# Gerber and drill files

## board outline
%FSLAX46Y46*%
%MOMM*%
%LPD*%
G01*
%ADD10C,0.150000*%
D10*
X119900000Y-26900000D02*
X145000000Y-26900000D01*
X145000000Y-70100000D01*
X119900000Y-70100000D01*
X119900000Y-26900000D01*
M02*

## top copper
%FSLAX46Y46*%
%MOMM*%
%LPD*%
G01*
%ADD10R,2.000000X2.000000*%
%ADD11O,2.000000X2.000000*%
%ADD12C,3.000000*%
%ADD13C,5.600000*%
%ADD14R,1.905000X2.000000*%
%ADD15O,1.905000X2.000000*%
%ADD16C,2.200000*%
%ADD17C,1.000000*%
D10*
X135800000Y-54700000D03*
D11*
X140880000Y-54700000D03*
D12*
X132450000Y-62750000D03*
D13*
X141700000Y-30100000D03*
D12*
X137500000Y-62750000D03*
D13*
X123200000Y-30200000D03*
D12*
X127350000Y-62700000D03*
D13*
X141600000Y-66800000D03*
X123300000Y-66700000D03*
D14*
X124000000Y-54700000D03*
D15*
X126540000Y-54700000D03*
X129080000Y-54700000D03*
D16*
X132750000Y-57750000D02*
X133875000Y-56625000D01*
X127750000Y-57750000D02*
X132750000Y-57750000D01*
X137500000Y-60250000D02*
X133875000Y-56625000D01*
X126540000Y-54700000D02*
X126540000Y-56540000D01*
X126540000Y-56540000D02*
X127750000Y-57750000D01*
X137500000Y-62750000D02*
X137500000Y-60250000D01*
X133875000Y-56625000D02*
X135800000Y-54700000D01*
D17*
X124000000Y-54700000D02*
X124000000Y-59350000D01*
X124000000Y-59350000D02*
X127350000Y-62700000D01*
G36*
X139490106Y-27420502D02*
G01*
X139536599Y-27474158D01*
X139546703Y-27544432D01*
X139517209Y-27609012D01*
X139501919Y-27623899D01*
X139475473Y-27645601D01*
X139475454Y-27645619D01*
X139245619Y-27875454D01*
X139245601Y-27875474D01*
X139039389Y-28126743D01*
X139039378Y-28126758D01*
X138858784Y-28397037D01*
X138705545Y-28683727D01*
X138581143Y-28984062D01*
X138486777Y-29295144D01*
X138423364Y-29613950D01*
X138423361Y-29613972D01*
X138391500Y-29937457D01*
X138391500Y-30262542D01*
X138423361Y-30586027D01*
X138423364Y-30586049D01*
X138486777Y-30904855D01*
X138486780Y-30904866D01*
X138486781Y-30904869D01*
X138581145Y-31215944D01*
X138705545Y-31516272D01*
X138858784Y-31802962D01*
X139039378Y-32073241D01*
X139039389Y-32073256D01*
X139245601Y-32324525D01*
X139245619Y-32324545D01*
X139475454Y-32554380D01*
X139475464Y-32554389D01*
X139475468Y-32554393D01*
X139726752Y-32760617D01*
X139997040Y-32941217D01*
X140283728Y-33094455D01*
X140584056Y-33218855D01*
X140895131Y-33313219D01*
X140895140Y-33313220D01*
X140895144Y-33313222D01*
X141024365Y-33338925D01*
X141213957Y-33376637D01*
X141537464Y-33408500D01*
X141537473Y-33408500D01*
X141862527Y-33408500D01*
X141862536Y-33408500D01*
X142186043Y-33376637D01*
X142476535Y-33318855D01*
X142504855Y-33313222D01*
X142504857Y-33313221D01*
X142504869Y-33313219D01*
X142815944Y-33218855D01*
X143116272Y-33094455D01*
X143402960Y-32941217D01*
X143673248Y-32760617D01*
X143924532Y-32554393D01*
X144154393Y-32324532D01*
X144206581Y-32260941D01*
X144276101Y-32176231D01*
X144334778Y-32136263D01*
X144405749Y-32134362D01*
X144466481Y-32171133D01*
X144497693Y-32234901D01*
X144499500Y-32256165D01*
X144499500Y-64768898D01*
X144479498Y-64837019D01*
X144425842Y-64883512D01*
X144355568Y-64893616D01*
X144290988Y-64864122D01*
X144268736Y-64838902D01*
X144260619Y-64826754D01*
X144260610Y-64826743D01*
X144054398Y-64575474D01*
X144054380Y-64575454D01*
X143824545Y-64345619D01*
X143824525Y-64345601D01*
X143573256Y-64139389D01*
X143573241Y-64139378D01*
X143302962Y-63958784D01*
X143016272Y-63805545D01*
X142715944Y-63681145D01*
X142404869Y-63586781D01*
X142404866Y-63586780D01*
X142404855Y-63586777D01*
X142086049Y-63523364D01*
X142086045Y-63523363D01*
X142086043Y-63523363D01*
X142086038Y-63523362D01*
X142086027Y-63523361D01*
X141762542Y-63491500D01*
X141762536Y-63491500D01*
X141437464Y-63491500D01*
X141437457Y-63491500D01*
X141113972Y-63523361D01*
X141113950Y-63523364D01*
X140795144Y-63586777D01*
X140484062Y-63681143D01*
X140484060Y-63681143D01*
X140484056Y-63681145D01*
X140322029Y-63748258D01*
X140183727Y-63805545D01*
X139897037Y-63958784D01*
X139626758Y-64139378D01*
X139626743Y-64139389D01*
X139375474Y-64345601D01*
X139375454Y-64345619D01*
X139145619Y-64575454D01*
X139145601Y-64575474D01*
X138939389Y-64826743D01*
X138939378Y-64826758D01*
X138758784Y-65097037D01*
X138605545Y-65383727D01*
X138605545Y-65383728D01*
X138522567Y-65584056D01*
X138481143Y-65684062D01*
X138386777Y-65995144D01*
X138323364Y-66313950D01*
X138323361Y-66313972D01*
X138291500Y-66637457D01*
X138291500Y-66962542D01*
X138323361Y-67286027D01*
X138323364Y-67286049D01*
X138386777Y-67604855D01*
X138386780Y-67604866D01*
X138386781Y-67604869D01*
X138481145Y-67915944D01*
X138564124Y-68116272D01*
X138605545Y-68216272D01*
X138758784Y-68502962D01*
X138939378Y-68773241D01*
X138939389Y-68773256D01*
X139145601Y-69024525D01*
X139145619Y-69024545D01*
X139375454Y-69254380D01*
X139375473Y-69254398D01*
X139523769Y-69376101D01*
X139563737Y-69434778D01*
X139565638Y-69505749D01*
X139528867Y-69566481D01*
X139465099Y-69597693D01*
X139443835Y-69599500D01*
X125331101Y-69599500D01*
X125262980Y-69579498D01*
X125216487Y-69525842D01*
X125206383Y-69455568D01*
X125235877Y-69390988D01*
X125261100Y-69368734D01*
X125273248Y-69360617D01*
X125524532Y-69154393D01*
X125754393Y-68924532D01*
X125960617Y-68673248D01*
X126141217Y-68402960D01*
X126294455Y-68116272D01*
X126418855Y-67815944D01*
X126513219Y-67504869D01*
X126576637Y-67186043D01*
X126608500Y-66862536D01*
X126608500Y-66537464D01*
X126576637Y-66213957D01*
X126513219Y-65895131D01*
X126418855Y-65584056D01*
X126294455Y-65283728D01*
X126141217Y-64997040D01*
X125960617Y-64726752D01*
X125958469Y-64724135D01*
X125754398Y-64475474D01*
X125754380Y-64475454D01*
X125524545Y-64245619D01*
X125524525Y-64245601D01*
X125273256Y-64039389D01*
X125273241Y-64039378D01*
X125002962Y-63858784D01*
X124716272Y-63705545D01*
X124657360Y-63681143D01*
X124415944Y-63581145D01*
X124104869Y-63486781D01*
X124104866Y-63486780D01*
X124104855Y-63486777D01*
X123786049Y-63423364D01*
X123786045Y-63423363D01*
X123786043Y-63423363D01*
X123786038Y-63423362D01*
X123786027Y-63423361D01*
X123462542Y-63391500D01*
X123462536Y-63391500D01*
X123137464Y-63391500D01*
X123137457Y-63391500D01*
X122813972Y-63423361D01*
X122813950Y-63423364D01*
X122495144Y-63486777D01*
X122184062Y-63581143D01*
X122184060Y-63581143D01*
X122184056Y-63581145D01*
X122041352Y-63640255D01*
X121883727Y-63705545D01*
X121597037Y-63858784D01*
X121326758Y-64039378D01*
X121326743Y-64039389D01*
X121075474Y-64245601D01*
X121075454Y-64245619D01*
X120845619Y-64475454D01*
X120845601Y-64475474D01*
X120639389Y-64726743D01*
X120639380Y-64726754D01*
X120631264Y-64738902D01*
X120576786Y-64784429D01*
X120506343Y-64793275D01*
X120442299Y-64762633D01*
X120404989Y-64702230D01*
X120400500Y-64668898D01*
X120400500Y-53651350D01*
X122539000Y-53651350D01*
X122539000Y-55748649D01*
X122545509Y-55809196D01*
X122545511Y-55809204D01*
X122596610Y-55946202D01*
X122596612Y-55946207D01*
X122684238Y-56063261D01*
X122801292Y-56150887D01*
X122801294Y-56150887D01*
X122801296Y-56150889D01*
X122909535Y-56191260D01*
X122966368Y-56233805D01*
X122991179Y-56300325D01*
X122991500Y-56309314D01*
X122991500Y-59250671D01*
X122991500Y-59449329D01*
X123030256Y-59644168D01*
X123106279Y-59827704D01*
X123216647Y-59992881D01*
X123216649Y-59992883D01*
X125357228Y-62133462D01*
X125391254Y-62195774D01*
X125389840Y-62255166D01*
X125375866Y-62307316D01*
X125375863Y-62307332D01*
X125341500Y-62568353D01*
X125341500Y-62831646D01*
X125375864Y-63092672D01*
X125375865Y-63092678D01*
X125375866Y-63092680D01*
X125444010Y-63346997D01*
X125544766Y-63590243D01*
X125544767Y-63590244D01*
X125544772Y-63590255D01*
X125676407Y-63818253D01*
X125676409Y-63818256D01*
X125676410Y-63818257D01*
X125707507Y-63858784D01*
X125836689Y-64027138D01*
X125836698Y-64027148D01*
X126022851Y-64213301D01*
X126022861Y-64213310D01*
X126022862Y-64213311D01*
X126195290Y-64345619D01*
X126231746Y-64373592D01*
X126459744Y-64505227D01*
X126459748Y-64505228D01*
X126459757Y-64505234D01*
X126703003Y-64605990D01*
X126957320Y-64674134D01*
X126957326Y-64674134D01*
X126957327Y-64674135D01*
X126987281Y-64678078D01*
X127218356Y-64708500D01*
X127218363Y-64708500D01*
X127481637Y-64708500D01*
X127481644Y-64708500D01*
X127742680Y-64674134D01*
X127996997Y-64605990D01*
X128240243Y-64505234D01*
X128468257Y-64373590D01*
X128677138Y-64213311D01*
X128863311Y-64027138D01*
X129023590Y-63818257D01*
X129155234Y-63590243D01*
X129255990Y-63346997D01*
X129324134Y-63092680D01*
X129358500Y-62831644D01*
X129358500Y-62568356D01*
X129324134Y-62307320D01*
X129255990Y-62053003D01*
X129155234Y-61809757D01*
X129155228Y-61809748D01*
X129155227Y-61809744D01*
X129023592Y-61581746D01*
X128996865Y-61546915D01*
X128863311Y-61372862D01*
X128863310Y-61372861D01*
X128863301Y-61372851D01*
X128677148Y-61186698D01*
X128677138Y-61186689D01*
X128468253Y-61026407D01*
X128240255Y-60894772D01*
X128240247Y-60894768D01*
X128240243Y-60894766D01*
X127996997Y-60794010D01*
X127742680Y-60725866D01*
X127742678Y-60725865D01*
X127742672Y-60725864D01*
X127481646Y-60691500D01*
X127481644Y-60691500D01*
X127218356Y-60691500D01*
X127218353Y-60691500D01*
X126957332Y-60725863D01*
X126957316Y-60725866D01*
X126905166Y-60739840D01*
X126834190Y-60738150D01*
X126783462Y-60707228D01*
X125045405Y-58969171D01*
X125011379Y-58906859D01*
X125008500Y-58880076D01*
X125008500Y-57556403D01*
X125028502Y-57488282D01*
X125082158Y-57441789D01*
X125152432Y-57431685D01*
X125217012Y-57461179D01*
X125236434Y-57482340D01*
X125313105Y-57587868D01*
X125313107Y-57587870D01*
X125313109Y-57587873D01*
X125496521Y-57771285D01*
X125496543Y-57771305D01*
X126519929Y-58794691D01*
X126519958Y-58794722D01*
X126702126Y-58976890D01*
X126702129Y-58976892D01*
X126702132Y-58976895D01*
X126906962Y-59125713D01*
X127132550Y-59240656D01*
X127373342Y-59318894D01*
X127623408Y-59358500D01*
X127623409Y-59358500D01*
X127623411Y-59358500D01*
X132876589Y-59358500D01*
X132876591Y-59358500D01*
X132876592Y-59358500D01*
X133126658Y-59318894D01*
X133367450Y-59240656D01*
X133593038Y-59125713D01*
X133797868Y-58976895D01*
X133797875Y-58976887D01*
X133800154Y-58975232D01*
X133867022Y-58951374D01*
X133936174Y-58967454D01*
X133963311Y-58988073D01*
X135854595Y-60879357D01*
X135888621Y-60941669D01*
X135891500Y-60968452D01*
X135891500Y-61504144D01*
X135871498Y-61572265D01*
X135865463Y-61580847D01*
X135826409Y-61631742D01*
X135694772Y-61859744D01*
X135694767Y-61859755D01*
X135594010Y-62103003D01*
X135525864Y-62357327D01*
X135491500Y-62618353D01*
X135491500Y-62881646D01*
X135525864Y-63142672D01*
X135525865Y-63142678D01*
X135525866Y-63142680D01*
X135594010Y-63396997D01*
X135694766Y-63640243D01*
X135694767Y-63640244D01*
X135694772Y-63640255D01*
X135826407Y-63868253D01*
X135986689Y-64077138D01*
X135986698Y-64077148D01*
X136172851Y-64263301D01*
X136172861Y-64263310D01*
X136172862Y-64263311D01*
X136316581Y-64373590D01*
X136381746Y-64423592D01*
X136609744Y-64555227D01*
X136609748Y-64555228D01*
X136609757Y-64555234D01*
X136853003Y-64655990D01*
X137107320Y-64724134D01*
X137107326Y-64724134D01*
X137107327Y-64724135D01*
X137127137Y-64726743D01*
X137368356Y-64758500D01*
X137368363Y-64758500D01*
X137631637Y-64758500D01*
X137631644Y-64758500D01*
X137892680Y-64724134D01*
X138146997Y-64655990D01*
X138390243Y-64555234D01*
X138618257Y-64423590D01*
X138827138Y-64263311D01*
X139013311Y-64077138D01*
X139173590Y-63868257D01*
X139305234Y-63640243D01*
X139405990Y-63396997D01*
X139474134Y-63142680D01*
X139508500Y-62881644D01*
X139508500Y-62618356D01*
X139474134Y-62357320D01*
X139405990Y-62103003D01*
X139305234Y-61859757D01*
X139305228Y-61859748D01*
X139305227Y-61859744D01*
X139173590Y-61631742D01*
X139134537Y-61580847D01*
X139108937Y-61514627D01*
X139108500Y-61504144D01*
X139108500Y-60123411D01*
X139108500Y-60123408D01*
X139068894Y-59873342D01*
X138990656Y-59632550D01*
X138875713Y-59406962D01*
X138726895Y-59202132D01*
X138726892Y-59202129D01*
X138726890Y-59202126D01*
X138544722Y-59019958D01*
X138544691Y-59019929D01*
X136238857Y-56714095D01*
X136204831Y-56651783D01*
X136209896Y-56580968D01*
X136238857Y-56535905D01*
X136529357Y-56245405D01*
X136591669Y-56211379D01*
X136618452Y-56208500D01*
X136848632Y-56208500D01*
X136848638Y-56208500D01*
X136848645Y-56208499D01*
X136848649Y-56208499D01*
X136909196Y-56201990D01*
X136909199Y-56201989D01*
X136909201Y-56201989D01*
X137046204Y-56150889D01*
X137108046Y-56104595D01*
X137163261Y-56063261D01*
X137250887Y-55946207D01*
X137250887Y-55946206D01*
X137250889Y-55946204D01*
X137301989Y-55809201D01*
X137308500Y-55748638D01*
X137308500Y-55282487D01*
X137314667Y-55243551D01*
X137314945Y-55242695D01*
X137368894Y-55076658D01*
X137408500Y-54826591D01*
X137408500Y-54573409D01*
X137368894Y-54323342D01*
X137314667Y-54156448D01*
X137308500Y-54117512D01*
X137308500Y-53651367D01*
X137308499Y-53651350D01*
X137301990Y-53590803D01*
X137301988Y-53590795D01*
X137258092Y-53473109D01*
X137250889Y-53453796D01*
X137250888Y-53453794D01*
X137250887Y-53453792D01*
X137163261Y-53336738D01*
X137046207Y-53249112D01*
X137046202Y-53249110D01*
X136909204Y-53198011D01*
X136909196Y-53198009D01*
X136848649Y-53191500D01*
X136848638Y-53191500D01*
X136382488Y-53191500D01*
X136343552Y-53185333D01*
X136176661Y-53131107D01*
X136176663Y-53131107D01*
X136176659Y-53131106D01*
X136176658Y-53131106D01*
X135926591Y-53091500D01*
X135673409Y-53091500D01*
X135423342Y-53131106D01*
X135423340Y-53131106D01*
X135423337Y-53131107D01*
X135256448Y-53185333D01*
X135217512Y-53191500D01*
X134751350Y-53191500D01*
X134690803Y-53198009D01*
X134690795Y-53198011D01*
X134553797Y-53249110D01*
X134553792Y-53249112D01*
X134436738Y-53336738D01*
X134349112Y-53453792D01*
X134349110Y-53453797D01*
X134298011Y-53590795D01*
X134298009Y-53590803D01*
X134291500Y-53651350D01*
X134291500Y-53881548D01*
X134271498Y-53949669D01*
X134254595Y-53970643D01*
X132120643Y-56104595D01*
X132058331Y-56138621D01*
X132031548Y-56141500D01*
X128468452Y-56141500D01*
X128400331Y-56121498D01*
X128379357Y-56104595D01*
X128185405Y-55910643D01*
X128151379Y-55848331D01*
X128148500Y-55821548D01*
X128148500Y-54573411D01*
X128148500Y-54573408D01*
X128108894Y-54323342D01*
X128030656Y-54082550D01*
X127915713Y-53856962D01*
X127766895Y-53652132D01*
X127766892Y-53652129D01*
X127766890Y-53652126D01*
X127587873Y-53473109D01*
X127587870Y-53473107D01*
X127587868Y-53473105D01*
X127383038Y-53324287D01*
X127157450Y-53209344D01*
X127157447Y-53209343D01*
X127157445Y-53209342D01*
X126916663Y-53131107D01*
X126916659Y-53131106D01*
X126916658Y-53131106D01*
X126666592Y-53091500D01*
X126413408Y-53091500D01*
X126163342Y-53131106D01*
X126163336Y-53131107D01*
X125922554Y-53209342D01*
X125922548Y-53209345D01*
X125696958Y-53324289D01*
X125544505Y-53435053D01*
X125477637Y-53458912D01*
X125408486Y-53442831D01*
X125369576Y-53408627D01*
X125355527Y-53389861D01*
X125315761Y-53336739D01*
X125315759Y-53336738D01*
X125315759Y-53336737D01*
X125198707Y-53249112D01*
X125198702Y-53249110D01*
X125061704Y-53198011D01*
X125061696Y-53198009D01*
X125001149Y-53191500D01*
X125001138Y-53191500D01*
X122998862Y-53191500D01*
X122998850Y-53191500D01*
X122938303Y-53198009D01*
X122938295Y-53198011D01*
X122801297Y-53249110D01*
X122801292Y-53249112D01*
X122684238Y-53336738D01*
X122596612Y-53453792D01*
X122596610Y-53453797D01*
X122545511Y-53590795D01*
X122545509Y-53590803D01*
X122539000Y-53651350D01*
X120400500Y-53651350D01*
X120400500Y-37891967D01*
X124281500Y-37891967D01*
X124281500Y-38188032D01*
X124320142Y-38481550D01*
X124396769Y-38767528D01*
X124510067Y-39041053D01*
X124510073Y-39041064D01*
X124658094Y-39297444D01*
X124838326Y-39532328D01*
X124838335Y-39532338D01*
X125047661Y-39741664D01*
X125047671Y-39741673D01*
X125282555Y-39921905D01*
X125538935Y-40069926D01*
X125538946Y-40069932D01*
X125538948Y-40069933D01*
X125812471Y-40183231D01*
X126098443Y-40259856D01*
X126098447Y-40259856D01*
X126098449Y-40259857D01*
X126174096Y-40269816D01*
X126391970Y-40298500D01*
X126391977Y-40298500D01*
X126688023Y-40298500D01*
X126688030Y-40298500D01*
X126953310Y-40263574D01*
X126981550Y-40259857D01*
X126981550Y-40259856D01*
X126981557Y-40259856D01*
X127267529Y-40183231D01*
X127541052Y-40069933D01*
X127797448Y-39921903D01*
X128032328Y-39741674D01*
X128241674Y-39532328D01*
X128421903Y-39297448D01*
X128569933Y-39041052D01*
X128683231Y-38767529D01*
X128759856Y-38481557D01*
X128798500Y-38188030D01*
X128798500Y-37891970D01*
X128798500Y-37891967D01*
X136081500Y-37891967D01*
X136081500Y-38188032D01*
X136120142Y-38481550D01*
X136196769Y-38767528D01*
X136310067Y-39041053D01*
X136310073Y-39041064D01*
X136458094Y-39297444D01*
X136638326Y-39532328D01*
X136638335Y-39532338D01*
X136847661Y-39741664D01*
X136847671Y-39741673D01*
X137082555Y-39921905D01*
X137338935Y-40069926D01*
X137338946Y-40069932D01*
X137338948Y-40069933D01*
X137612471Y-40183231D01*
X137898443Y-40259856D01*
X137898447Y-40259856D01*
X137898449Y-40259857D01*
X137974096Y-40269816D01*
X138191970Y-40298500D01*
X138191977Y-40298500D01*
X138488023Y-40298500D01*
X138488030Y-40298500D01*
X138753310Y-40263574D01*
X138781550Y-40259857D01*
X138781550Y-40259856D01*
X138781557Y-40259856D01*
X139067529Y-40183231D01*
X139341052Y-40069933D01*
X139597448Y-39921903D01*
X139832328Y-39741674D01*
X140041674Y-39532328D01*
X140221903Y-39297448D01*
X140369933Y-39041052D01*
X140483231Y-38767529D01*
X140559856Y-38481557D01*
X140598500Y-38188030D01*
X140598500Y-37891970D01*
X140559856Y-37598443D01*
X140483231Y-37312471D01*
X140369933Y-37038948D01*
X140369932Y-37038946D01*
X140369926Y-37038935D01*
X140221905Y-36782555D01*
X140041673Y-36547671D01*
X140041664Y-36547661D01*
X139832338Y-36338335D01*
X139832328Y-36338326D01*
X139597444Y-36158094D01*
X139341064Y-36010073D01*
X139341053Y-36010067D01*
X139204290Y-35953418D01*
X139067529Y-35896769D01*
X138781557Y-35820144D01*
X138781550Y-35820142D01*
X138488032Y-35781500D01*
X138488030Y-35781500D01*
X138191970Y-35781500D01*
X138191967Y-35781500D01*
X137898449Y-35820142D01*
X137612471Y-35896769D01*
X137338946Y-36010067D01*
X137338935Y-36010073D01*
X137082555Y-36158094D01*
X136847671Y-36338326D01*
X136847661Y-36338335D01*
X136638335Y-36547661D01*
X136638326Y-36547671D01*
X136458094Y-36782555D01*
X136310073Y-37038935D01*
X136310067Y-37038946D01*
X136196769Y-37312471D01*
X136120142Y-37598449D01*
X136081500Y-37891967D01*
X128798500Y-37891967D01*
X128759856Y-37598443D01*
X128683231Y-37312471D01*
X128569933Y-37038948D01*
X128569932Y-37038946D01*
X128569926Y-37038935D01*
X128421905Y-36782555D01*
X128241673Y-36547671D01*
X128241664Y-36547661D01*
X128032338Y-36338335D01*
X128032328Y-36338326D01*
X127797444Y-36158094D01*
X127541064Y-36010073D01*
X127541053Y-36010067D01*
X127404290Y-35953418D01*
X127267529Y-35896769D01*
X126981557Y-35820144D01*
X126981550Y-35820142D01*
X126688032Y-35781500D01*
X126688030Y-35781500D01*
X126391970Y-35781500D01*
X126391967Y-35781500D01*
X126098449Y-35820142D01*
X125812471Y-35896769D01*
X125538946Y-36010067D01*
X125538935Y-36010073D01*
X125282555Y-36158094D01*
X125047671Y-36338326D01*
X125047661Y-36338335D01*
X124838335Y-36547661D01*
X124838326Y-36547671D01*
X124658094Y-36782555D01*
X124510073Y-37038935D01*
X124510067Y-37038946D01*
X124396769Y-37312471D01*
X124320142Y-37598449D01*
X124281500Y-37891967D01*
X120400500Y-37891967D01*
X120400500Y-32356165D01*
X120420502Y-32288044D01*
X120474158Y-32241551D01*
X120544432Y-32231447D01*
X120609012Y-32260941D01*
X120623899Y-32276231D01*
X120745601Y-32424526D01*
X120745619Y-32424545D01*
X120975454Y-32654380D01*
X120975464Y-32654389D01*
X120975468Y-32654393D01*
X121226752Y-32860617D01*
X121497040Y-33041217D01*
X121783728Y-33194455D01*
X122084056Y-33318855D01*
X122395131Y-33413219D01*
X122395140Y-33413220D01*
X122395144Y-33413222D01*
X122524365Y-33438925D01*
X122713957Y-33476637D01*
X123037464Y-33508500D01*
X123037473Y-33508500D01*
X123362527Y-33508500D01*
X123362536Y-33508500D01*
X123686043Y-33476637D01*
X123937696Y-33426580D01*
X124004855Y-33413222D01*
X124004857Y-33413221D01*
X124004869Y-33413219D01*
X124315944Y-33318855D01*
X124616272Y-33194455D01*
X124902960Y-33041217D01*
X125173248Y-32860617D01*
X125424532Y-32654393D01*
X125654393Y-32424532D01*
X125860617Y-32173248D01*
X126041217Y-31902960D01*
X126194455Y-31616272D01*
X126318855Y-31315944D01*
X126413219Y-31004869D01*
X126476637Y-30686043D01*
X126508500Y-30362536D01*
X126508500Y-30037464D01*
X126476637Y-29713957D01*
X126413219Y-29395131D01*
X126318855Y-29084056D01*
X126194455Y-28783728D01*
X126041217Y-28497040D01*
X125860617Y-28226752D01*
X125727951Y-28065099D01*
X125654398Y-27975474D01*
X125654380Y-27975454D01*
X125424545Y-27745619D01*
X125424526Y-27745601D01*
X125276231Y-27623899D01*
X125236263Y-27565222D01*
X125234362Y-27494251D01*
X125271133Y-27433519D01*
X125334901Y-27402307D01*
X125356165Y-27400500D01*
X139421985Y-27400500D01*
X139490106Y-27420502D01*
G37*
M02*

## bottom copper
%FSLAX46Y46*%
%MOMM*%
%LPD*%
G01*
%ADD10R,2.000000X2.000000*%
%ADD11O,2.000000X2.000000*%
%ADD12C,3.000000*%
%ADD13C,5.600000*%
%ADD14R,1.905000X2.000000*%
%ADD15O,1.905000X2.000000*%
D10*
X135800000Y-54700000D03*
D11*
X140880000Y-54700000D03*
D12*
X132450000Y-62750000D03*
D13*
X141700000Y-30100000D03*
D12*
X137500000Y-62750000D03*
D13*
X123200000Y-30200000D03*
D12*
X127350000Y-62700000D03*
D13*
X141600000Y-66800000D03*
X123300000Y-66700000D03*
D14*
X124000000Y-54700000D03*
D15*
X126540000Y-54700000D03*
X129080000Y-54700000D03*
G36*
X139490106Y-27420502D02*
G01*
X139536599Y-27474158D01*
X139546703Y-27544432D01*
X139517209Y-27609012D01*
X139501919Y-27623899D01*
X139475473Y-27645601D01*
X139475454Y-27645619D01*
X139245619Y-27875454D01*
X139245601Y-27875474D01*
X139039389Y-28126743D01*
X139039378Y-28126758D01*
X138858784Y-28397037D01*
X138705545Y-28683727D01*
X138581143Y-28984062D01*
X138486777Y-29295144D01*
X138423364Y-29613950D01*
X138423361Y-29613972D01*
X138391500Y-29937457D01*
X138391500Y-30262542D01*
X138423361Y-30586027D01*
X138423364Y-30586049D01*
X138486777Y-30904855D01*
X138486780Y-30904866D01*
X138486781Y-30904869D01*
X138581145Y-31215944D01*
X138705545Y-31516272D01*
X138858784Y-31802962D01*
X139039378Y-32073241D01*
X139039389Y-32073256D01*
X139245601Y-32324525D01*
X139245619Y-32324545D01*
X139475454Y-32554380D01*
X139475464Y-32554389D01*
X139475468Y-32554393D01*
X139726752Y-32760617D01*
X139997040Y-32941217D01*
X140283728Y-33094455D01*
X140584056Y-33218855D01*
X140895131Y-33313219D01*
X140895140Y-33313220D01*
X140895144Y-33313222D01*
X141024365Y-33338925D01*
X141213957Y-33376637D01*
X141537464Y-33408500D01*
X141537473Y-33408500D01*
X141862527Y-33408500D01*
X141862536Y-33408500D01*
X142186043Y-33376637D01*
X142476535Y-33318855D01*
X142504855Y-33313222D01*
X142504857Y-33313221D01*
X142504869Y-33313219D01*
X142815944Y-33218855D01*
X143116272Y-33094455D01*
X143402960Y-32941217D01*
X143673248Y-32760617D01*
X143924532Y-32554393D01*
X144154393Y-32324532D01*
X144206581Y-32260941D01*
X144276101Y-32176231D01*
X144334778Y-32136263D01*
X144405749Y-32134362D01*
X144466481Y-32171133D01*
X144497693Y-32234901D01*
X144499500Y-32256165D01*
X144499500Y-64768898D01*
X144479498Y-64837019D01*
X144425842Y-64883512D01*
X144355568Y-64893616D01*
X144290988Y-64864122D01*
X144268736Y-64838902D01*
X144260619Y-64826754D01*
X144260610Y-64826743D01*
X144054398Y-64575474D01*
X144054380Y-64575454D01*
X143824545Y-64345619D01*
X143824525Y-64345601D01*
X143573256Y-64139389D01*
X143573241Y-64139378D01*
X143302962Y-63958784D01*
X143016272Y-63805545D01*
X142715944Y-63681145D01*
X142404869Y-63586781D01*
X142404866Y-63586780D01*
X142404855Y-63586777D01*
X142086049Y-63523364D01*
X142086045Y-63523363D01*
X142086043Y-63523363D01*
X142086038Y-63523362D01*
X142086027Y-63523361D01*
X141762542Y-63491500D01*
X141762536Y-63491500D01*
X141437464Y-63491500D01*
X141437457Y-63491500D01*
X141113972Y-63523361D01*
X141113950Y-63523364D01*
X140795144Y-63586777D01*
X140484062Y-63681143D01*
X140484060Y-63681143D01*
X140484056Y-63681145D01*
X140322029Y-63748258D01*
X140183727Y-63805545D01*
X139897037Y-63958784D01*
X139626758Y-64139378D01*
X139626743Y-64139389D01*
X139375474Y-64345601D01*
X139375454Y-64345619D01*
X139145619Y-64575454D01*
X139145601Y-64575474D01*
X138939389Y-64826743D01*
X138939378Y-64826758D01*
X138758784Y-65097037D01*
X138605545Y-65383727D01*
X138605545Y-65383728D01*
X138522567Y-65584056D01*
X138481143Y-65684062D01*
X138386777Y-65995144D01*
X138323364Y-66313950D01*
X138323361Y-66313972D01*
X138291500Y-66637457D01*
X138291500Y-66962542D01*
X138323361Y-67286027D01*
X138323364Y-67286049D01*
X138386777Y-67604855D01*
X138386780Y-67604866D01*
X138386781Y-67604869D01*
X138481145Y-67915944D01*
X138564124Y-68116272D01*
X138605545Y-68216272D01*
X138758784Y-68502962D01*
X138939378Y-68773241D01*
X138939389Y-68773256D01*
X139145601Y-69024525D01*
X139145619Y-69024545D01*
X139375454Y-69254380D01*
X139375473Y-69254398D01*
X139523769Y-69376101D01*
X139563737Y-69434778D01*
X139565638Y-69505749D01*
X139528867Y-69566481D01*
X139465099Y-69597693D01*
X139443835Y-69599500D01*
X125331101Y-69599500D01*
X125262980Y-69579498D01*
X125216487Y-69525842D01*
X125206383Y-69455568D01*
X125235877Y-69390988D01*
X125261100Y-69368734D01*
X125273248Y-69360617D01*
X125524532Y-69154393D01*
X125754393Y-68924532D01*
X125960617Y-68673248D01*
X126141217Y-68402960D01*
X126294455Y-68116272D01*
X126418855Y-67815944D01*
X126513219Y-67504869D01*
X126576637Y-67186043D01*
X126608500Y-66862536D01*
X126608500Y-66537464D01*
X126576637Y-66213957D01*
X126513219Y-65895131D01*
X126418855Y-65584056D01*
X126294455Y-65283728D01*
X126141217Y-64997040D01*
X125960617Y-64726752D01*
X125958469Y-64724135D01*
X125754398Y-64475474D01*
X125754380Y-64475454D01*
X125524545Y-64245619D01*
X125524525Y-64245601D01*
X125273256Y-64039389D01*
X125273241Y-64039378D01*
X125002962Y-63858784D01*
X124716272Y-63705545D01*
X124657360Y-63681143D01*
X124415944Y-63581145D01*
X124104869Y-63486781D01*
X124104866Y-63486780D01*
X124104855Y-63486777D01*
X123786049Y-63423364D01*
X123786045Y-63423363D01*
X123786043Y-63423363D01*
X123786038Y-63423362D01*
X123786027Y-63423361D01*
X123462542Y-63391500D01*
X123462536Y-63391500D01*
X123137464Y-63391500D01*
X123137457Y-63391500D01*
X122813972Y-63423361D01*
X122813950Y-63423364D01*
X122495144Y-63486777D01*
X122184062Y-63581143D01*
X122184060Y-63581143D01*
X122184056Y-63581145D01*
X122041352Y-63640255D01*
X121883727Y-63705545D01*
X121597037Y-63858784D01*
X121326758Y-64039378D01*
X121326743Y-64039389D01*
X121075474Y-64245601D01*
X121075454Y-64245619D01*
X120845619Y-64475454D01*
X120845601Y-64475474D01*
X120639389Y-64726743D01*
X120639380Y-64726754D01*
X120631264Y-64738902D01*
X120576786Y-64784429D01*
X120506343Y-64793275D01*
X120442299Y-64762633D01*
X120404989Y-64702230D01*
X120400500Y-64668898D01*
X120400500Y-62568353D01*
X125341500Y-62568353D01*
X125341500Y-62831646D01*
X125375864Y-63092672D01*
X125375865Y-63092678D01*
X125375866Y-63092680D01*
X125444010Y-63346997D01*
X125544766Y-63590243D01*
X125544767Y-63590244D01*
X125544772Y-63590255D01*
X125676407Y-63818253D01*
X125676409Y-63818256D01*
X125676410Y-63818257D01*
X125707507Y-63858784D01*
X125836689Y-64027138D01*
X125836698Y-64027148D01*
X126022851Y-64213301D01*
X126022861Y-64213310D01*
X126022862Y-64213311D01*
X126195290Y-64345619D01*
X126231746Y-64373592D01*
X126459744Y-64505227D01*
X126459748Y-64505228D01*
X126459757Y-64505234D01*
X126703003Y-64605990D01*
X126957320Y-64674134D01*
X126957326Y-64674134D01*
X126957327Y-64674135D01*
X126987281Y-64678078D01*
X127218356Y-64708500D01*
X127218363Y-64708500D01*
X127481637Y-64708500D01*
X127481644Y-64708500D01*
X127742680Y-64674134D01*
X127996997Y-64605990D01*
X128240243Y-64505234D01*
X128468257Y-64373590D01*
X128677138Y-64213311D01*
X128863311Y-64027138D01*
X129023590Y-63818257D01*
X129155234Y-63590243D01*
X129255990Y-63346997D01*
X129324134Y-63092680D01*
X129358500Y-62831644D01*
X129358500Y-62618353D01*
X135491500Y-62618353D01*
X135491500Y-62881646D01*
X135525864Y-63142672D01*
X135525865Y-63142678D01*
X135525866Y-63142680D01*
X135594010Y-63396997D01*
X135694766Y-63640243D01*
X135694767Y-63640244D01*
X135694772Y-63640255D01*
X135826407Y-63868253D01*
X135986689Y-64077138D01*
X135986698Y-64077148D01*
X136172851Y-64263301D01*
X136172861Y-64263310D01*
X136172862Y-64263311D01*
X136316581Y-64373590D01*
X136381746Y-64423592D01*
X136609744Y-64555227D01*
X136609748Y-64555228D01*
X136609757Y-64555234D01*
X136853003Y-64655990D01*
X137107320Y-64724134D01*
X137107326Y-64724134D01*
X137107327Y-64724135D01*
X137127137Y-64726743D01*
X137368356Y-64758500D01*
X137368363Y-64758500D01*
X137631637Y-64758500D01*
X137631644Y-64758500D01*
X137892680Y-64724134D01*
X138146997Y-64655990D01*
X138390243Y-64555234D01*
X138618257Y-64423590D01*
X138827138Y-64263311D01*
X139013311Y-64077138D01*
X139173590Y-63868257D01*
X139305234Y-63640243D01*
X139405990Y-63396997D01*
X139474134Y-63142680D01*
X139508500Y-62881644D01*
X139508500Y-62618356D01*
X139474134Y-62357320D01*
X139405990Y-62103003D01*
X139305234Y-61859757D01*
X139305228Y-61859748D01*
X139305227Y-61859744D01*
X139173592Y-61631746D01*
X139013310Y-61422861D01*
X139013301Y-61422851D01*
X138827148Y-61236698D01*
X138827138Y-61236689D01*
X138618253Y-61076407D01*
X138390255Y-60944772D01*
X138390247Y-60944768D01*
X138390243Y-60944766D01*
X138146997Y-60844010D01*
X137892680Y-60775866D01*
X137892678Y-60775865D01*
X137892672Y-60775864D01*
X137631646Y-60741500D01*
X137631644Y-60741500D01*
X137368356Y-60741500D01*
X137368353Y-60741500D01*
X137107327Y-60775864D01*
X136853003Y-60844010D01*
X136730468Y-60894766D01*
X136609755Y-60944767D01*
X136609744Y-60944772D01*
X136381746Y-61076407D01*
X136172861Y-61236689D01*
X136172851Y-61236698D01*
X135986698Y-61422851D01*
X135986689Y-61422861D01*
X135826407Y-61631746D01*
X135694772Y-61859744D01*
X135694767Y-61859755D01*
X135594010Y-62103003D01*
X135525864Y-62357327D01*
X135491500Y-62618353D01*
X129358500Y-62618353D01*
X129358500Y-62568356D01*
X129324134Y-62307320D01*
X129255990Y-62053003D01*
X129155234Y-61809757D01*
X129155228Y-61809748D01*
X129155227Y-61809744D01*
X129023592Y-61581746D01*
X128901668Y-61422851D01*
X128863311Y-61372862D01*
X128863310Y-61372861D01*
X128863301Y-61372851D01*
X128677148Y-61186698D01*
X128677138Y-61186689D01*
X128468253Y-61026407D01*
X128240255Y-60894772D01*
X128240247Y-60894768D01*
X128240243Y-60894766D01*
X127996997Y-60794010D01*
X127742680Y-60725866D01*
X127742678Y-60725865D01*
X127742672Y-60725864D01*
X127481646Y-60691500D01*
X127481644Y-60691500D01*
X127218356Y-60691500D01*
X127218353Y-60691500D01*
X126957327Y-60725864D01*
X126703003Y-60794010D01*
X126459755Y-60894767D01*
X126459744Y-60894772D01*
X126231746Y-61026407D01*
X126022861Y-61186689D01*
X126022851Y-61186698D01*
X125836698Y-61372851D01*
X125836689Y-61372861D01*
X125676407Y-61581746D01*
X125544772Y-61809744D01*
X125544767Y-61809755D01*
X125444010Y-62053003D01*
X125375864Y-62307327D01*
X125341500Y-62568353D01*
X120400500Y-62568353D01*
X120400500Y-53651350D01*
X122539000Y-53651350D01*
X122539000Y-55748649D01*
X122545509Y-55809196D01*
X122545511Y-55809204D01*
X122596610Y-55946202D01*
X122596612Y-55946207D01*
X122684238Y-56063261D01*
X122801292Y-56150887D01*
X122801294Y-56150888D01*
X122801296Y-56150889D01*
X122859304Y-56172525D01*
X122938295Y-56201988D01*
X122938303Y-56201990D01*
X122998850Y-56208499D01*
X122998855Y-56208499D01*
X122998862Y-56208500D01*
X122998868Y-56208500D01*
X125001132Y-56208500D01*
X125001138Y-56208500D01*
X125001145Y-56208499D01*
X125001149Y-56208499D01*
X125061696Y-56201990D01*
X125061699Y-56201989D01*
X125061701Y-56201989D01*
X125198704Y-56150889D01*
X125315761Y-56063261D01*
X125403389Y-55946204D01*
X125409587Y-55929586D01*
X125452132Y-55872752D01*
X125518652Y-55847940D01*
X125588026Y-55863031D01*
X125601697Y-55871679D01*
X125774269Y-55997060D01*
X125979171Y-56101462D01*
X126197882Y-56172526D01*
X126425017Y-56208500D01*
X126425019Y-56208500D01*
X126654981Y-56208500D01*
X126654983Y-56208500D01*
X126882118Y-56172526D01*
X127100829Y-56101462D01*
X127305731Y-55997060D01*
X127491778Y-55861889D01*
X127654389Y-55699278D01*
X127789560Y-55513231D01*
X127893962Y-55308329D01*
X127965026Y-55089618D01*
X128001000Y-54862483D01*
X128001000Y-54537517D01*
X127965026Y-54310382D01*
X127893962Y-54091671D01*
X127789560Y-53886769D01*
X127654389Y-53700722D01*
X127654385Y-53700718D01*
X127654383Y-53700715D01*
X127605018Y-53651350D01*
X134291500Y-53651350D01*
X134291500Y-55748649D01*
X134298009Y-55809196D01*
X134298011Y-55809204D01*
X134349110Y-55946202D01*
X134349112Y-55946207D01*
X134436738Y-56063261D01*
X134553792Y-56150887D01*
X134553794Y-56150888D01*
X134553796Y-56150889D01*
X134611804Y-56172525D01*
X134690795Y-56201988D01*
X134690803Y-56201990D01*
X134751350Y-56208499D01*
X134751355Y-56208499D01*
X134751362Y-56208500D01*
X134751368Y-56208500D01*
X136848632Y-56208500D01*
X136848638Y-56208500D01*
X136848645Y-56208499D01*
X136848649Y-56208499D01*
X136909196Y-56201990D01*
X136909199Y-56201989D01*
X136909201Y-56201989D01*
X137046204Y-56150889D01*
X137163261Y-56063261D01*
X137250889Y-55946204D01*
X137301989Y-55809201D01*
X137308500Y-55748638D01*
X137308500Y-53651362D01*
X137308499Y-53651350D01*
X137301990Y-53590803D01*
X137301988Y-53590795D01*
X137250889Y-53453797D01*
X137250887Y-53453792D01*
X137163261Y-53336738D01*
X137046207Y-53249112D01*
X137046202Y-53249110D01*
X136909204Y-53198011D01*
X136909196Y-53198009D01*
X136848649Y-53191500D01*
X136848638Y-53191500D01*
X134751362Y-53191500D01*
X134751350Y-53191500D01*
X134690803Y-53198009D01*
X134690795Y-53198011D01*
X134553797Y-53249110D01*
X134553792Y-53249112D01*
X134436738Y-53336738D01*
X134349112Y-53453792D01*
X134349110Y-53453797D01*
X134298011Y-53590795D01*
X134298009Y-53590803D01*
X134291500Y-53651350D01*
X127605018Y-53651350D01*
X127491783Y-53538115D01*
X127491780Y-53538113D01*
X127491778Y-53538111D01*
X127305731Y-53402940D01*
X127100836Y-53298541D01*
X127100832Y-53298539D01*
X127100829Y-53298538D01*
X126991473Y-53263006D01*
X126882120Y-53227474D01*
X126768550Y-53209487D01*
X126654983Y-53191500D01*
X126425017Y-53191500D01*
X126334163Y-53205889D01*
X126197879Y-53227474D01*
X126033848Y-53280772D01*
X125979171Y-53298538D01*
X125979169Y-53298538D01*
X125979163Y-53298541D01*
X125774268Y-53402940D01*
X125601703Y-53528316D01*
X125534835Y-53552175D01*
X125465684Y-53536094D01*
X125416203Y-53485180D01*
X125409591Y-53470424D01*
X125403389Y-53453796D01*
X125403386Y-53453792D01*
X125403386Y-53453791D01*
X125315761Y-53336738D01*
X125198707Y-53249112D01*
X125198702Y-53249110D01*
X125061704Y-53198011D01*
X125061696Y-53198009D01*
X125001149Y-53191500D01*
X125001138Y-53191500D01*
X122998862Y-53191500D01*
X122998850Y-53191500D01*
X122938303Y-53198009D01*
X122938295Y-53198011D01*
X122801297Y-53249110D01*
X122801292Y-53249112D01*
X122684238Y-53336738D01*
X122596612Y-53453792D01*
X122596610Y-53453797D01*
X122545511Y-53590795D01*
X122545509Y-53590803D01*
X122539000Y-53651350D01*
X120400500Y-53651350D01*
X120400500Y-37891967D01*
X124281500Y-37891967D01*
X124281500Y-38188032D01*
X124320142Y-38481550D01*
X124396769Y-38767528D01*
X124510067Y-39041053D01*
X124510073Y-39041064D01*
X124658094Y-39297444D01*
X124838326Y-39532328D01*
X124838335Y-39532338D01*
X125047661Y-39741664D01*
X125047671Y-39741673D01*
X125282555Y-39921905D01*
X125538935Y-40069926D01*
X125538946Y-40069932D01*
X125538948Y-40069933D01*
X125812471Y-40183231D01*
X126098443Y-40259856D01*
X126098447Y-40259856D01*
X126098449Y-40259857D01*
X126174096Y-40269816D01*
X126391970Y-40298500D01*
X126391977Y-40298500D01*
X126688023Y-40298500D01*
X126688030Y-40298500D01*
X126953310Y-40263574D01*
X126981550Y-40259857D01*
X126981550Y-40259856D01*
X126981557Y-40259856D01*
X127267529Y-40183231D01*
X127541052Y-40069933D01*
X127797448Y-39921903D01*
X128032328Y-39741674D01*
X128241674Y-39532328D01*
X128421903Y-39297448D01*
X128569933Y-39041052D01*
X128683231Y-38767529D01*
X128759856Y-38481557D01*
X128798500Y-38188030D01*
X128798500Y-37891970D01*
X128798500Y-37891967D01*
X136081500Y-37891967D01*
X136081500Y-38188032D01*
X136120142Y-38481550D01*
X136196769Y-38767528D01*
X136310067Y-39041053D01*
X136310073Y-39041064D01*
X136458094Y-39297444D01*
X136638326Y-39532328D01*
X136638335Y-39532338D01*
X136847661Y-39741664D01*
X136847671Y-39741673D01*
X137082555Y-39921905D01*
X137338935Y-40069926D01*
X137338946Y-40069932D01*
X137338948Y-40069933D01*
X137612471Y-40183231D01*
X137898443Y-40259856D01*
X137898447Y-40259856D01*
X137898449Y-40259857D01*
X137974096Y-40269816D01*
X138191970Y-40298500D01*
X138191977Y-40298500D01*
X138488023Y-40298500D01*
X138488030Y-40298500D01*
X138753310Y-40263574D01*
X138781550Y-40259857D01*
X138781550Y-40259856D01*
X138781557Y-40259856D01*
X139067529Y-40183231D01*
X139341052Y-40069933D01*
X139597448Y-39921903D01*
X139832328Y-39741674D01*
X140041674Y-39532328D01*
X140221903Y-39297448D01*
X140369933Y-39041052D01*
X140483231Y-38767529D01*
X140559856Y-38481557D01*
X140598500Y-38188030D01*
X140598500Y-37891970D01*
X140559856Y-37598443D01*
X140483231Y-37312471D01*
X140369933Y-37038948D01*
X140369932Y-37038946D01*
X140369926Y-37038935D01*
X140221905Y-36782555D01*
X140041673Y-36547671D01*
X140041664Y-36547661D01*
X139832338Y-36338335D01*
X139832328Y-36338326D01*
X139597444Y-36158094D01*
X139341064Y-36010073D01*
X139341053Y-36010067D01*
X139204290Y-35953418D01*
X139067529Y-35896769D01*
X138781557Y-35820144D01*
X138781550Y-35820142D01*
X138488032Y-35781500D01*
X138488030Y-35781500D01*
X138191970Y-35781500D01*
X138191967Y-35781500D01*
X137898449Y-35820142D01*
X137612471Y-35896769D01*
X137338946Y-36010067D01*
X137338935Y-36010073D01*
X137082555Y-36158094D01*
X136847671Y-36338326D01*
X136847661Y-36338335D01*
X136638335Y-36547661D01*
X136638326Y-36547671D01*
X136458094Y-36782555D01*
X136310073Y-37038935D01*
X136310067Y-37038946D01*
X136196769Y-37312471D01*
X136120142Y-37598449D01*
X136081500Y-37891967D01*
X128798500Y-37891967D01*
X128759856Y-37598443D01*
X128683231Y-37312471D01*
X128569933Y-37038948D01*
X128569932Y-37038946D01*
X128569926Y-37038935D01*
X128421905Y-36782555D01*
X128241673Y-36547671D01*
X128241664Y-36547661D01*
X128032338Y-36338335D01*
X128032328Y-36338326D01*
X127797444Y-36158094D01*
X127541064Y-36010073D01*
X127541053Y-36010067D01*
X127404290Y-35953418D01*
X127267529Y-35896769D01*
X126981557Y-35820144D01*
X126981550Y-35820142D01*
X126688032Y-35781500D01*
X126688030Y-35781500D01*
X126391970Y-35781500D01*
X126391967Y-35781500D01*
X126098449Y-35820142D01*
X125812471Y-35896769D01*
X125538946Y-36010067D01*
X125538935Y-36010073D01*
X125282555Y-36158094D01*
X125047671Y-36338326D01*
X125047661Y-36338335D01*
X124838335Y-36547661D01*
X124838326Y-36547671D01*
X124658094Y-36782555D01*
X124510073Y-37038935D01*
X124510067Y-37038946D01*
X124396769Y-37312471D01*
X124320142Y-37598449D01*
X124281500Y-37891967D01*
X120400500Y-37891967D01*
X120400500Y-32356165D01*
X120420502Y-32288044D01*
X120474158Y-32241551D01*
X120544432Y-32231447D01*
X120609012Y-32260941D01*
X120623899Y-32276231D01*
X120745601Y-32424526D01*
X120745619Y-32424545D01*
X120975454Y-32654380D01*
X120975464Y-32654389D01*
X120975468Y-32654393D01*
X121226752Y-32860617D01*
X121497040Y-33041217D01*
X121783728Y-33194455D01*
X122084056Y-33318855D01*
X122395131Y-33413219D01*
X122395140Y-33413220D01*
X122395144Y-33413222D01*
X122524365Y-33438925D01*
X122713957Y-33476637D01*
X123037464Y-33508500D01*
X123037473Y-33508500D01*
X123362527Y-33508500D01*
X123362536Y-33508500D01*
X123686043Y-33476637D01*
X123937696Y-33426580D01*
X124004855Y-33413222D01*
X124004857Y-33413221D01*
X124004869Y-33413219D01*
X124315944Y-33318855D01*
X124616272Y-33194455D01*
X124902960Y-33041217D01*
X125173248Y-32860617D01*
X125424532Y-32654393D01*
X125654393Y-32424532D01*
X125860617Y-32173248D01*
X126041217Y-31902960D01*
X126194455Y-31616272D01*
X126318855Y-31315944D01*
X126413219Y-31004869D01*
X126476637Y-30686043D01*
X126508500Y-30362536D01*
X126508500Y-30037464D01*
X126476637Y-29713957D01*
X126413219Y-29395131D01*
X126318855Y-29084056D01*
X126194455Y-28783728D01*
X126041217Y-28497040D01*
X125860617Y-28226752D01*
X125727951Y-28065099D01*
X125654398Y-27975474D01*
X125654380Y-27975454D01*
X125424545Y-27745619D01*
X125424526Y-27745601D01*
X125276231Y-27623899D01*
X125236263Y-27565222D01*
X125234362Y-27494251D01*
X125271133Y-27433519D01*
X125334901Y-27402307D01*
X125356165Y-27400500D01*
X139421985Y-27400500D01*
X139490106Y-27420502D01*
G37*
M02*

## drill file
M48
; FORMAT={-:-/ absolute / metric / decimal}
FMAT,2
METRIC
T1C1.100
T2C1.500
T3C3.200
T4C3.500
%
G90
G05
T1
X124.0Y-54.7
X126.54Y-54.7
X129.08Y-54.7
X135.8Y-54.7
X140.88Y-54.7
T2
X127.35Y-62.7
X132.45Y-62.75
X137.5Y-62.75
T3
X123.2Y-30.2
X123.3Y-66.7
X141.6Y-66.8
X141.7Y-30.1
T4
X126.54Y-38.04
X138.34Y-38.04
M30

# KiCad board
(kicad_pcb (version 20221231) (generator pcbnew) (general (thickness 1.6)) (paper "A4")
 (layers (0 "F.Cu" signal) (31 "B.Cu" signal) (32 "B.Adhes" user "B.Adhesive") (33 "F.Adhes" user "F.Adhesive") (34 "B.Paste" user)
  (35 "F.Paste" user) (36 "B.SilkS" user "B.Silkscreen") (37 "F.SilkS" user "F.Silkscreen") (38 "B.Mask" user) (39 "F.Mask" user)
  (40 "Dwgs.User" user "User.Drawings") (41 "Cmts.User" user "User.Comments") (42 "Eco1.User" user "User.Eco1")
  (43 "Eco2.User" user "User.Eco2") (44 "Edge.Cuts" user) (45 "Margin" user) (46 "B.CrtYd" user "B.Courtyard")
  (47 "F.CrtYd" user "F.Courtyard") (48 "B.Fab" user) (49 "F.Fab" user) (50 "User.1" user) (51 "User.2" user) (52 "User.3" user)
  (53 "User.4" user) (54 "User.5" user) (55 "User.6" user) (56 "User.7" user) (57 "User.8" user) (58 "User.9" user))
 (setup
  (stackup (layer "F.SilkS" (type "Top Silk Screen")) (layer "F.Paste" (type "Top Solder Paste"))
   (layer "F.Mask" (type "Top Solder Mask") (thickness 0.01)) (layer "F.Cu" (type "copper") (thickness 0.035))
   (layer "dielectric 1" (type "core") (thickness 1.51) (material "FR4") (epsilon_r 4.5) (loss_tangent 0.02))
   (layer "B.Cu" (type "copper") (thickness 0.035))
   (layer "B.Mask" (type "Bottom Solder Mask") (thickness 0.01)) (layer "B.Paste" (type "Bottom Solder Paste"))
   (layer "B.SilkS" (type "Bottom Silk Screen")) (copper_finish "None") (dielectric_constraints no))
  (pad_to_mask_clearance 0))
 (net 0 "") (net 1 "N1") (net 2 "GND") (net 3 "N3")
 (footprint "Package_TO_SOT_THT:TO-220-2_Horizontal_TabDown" (layer "F.Cu") (at 135.8 54.7)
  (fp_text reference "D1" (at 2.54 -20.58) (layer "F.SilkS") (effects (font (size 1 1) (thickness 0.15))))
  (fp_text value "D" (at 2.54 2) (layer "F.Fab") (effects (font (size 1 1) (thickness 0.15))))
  (pad "" np_thru_hole oval locked (at 2.54 -16.66) (size 3.5 3.5) (drill 3.5) (layers *.Cu *.Mask))
  (pad "1" thru_hole rect locked (at 0 0) (size 2 2) (drill 1.1) (layers *.Cu *.Mask) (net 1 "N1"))
  (pad "2" thru_hole oval locked (at 5.08 0) (size 2 2) (drill 1.1) (layers *.Cu *.Mask) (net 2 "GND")))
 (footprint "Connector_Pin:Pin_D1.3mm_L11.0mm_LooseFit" (layer "F.Cu") (at 132.45 62.75)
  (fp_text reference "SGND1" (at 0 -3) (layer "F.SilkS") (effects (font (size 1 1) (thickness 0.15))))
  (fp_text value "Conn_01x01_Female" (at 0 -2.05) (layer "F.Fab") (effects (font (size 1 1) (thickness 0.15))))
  (pad "1" thru_hole circle locked (at 0 0) (size 3 3) (drill 1.5) (layers *.Cu *.Mask) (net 2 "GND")))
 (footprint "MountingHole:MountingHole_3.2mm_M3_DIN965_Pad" (layer "F.Cu") (at 141.7 30.1)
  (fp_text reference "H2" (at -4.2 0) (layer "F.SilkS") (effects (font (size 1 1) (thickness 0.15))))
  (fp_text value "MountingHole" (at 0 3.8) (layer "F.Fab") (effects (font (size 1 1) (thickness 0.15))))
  (pad "1" thru_hole circle locked (at 0 0) (size 5.6 5.6) (drill 3.2) (layers *.Cu *.Mask)))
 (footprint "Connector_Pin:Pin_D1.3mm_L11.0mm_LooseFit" (layer "F.Cu") (at 137.5 62.75)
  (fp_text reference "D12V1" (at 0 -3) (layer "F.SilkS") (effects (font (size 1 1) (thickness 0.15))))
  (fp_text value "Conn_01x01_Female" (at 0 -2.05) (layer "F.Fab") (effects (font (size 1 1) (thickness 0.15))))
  (pad "1" thru_hole circle locked (at 0 0) (size 3 3) (drill 1.5) (layers *.Cu *.Mask) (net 1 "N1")))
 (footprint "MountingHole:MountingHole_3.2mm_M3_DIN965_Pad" (layer "F.Cu") (at 123.2 30.2)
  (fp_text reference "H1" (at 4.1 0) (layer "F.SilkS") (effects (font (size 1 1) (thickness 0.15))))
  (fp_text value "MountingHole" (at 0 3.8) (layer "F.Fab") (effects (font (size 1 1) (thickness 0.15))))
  (pad "1" thru_hole circle locked (at 0 0) (size 5.6 5.6) (drill 3.2) (layers *.Cu *.Mask)))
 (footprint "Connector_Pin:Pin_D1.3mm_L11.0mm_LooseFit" (layer "F.Cu") (at 127.35 62.7)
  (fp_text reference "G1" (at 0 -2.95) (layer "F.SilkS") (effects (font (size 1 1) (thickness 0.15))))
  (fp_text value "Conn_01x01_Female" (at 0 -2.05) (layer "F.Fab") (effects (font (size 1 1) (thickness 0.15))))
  (pad "1" thru_hole circle locked (at 0 0) (size 3 3) (drill 1.5) (layers *.Cu *.Mask) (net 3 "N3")))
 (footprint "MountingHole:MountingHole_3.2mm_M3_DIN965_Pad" (layer "F.Cu") (at 141.6 66.8)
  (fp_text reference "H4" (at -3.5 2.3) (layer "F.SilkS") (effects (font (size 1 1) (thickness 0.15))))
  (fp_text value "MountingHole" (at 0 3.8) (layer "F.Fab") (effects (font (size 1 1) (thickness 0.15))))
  (pad "1" thru_hole circle locked (at 0 0) (size 5.6 5.6) (drill 3.2) (layers *.Cu *.Mask)))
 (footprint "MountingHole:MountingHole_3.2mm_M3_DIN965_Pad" (layer "F.Cu") (at 123.3 66.7)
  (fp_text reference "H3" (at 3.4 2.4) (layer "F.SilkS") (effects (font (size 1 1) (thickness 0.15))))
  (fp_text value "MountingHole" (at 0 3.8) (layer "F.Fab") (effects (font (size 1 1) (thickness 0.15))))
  (pad "1" thru_hole circle locked (at 0 0) (size 5.6 5.6) (drill 3.2) (layers *.Cu *.Mask)))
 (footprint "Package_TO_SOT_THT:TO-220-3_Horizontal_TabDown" (layer "F.Cu") (at 124 54.7) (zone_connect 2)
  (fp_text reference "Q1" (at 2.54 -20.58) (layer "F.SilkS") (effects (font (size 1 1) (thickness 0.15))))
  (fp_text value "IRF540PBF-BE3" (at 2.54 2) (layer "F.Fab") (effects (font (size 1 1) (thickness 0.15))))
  (pad "" np_thru_hole oval locked (at 2.54 -16.66) (size 3.5 3.5) (drill 3.5) (layers *.Cu *.Mask))
  (pad "1" thru_hole rect locked (at 0 0) (size 1.905 2) (drill 1.1) (layers *.Cu *.Mask) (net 3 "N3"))
  (pad "2" thru_hole oval locked (at 2.54 0) (size 1.905 2) (drill 1.1) (layers *.Cu *.Mask) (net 1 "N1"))
  (pad "3" thru_hole oval locked (at 5.08 0) (size 1.905 2) (drill 1.1) (layers *.Cu *.Mask) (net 2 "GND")))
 (gr_rect (start 119.9 26.9) (end 145 70.1) (stroke (width 0.15) (type default)) (fill none) (layer "Edge.Cuts"))
 (segment (start 132.75 57.75) (end 133.875 56.625) (width 2.2) (layer "F.Cu") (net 1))
 (segment (start 127.75 57.75) (end 132.75 57.75) (width 2.2) (layer "F.Cu") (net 1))
 (segment (start 137.5 60.25) (end 133.875 56.625) (width 2.2) (layer "F.Cu") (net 1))
 (segment (start 126.54 54.7) (end 126.54 56.54) (width 2.2) (layer "F.Cu") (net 1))
 (segment (start 126.54 56.54) (end 127.75 57.75) (width 2.2) (layer "F.Cu") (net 1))
 (segment (start 137.5 62.75) (end 137.5 60.25) (width 2.2) (layer "F.Cu") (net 1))
 (segment (start 133.875 56.625) (end 135.8 54.7) (width 2.2) (layer "F.Cu") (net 1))
 (segment (start 124 54.7) (end 124 59.35) (width 1) (layer "F.Cu") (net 3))
 (segment (start 124 59.35) (end 127.35 62.7) (width 1) (layer "F.Cu") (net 3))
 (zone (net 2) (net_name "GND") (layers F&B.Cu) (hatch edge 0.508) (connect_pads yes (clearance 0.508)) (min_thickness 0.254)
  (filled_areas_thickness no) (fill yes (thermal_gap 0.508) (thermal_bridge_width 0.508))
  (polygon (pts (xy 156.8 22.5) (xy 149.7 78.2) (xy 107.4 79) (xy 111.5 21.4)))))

